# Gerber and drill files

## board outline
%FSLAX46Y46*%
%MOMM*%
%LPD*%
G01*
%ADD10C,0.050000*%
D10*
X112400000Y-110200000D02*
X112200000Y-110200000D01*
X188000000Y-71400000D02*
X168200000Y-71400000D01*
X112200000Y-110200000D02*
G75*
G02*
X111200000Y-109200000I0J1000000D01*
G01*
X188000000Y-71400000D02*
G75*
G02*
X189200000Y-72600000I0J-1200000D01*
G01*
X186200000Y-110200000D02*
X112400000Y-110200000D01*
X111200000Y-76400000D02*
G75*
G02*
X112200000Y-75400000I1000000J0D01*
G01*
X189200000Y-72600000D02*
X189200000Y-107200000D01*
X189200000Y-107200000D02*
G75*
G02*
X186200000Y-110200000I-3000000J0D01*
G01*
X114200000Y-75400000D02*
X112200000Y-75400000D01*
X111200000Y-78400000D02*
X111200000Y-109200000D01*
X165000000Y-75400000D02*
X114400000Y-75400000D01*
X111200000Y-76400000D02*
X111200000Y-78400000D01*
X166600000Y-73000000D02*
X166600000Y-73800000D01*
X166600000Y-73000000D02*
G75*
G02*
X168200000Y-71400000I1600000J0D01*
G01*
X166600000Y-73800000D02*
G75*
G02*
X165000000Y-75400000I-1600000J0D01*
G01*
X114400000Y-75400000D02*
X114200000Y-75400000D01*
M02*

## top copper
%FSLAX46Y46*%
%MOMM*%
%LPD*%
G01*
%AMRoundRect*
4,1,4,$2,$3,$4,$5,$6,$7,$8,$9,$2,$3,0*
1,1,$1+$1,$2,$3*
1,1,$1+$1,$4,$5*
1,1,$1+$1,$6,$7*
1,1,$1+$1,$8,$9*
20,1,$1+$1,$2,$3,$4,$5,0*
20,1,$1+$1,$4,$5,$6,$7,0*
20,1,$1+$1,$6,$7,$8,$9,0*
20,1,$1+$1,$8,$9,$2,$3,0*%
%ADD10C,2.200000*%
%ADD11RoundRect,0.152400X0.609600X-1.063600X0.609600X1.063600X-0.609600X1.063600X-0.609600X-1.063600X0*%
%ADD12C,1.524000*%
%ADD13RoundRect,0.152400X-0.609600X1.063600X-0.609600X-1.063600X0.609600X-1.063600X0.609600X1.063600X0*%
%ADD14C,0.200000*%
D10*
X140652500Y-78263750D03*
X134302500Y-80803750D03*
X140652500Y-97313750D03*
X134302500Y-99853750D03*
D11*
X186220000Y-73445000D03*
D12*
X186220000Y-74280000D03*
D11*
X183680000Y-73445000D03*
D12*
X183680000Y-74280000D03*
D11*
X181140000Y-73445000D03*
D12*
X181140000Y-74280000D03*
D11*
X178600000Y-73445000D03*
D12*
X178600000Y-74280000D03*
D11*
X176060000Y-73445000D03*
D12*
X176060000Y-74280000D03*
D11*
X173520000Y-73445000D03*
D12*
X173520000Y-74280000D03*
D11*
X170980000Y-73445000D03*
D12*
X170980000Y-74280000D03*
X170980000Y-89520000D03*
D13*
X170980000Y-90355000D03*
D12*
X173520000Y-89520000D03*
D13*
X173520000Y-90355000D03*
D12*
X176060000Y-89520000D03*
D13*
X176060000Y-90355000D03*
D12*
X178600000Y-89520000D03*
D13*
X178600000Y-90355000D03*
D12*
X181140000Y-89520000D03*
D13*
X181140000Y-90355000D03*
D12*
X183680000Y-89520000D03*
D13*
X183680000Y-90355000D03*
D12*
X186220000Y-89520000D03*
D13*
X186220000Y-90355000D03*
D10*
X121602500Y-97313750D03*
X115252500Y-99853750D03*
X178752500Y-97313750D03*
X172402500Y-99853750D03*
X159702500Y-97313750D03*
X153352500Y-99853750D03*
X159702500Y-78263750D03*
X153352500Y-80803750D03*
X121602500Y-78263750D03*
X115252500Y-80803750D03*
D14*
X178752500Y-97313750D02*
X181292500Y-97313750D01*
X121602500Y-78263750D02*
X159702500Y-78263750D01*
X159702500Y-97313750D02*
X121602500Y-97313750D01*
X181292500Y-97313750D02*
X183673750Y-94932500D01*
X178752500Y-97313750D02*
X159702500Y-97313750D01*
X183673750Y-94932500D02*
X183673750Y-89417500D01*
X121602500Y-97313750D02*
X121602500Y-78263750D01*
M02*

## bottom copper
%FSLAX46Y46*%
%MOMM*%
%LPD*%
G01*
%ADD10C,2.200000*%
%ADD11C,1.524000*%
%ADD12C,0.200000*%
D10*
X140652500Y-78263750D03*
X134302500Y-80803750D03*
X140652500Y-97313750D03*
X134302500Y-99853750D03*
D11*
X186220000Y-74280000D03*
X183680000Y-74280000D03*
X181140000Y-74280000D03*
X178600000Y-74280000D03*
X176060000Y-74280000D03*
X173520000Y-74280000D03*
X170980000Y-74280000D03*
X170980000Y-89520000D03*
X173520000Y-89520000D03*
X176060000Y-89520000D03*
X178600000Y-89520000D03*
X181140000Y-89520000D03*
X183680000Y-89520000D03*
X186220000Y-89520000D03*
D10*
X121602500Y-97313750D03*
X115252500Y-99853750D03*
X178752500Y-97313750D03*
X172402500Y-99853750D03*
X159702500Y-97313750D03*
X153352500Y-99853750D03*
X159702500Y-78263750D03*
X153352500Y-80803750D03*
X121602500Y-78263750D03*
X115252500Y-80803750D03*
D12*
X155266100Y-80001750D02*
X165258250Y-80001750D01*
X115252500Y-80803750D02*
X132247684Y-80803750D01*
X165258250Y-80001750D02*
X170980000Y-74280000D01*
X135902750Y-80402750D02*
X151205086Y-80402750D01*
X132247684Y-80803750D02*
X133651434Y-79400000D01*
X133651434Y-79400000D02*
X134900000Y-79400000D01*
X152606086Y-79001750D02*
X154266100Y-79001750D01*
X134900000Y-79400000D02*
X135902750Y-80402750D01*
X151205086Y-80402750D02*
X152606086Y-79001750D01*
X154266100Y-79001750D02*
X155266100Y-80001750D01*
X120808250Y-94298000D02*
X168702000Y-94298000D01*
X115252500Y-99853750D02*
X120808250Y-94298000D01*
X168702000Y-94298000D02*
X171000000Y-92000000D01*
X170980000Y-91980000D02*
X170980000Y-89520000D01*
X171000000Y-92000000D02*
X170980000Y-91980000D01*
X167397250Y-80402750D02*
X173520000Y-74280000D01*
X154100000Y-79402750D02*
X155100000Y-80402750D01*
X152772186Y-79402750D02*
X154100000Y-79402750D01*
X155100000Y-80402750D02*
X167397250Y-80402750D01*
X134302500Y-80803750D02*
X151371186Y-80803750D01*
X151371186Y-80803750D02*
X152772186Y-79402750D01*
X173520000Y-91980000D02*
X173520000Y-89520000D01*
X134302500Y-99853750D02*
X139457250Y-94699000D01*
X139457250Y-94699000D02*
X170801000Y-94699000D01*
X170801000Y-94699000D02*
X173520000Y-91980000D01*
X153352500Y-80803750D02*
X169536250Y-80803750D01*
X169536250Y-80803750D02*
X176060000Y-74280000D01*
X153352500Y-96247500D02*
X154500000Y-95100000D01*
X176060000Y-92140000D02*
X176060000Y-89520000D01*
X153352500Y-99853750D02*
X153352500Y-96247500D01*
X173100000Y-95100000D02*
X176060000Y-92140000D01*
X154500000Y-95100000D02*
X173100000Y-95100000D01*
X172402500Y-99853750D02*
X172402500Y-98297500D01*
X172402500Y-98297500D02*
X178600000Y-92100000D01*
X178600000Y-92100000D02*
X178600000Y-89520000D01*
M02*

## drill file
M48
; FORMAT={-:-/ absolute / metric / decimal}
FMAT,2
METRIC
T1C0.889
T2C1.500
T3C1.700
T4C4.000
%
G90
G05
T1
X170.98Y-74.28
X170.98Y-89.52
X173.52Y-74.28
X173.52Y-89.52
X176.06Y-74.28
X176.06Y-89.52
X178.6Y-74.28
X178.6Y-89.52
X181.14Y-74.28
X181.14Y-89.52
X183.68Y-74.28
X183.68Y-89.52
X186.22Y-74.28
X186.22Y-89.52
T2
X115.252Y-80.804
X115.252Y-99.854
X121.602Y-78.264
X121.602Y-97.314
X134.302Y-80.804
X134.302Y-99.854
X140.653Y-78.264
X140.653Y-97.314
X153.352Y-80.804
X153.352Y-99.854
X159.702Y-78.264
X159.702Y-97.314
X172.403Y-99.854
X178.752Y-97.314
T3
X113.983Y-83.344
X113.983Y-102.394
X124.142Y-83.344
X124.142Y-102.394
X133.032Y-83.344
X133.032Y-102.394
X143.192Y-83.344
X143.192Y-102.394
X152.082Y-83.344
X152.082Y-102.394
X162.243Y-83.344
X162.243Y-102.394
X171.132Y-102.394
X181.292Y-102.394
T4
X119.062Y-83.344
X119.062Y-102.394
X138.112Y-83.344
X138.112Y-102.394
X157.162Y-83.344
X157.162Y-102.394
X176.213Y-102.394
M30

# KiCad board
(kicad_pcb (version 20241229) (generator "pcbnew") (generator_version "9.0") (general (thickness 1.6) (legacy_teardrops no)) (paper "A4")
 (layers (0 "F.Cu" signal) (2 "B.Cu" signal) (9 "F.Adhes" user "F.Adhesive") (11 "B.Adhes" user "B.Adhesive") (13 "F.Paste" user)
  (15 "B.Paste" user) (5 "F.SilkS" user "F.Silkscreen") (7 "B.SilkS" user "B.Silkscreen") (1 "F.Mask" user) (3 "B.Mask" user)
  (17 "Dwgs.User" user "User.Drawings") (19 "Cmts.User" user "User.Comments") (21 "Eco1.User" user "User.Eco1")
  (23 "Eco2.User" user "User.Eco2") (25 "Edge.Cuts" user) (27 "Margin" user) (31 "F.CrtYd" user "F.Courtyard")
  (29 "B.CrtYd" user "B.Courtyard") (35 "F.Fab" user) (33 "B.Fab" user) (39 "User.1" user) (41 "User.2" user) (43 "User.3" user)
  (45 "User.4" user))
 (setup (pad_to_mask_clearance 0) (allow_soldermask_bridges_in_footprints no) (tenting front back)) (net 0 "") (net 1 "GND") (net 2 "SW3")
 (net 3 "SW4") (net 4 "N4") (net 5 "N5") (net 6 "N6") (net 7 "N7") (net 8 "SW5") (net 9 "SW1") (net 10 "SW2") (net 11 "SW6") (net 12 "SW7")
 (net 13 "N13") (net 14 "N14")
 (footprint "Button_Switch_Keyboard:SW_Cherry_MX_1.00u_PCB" (layer "F.Cu") (at 140.6525 78.26375)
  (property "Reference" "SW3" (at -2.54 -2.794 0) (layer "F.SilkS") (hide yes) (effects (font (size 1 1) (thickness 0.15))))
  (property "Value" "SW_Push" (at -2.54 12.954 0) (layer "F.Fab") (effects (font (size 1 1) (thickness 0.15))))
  (pad "" np_thru_hole circle (at -7.62 5.08) (size 1.7 1.7) (drill 1.7) (layers "*.Cu" "*.Mask"))
  (pad "" np_thru_hole circle (at -2.54 5.08) (size 4 4) (drill 4) (layers "*.Cu" "*.Mask"))
  (pad "" np_thru_hole circle (at 2.54 5.08) (size 1.7 1.7) (drill 1.7) (layers "*.Cu" "*.Mask"))
  (pad "1" thru_hole circle (at 0 0) (size 2.2 2.2) (drill 1.5) (layers "*.Cu" "*.Mask") (remove_unused_layers no) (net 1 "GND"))
  (pad "2" thru_hole circle (at -6.35 2.54) (size 2.2 2.2) (drill 1.5) (layers "*.Cu" "*.Mask") (remove_unused_layers no) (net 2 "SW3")))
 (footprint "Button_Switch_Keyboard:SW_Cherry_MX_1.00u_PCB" (layer "F.Cu") (at 140.6525 97.31375)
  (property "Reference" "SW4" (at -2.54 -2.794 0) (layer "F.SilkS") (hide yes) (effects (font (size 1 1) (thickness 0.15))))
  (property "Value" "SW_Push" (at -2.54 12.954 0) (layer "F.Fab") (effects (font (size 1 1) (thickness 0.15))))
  (pad "" np_thru_hole circle (at -7.62 5.08) (size 1.7 1.7) (drill 1.7) (layers "*.Cu" "*.Mask"))
  (pad "" np_thru_hole circle (at -2.54 5.08) (size 4 4) (drill 4) (layers "*.Cu" "*.Mask"))
  (pad "" np_thru_hole circle (at 2.54 5.08) (size 1.7 1.7) (drill 1.7) (layers "*.Cu" "*.Mask"))
  (pad "1" thru_hole circle (at 0 0) (size 2.2 2.2) (drill 1.5) (layers "*.Cu" "*.Mask") (remove_unused_layers no) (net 1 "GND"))
  (pad "2" thru_hole circle (at -6.35 2.54) (size 2.2 2.2) (drill 1.5) (layers "*.Cu" "*.Mask") (remove_unused_layers no) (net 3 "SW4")))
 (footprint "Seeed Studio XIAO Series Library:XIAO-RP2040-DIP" (layer "F.Cu") (at 178.6 81.9 -90)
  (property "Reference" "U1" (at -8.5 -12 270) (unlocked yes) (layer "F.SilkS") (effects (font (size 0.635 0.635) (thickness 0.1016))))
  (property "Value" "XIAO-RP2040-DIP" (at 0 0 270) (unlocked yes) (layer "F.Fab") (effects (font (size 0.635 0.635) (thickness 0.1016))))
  (pad "1" smd roundrect (at -8.455 -7.62 90) (size 2.432 1.524) (layers "F.Cu" "F.Mask") (roundrect_rratio 0.1) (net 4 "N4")
   (thermal_bridge_angle 45))
  (pad "1" thru_hole circle (at -7.62 -7.62 90) (size 1.524 1.524) (drill 0.889) (layers "*.Cu" "*.Mask") (remove_unused_layers no)
   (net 4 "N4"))
  (pad "2" smd roundrect (at -8.455 -5.08 90) (size 2.432 1.524) (layers "F.Cu" "F.Mask") (roundrect_rratio 0.1) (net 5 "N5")
   (thermal_bridge_angle 45))
  (pad "2" thru_hole circle (at -7.62 -5.08 90) (size 1.524 1.524) (drill 0.889) (layers "*.Cu" "*.Mask") (remove_unused_layers no)
   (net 5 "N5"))
  (pad "3" smd roundrect (at -8.455 -2.54 90) (size 2.432 1.524) (layers "F.Cu" "F.Mask") (roundrect_rratio 0.1) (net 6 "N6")
   (thermal_bridge_angle 45))
  (pad "3" thru_hole circle (at -7.62 -2.54 90) (size 1.524 1.524) (drill 0.889) (layers "*.Cu" "*.Mask") (remove_unused_layers no)
   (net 6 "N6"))
  (pad "4" smd roundrect (at -8.455 0 90) (size 2.432 1.524) (layers "F.Cu" "F.Mask") (roundrect_rratio 0.1) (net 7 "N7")
   (thermal_bridge_angle 45))
  (pad "4" thru_hole circle (at -7.62 0 90) (size 1.524 1.524) (drill 0.889) (layers "*.Cu" "*.Mask") (remove_unused_layers no) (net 7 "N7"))
  (pad "5" smd roundrect (at -8.455 2.54 90) (size 2.432 1.524) (layers "F.Cu" "F.Mask") (roundrect_rratio 0.1) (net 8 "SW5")
   (thermal_bridge_angle 45))
  (pad "5" thru_hole circle (at -7.62 2.54 90) (size 1.524 1.524) (drill 0.889) (layers "*.Cu" "*.Mask") (remove_unused_layers no)
   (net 8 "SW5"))
  (pad "6" smd roundrect (at -8.455 5.08 90) (size 2.432 1.524) (layers "F.Cu" "F.Mask") (roundrect_rratio 0.1) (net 2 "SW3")
   (thermal_bridge_angle 45))
  (pad "6" thru_hole circle (at -7.62 5.08 90) (size 1.524 1.524) (drill 0.889) (layers "*.Cu" "*.Mask") (remove_unused_layers no)
   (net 2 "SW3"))
  (pad "7" smd roundrect (at -8.455 7.62 90) (size 2.432 1.524) (layers "F.Cu" "F.Mask") (roundrect_rratio 0.1) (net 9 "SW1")
   (thermal_bridge_angle 45))
  (pad "7" thru_hole circle (at -7.62 7.62 90) (size 1.524 1.524) (drill 0.889) (layers "*.Cu" "*.Mask") (remove_unused_layers no)
   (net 9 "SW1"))
  (pad "8" thru_hole circle (at 7.62 7.62 270) (size 1.524 1.524) (drill 0.889) (layers "*.Cu" "*.Mask") (remove_unused_layers no)
   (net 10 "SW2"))
  (pad "8" smd roundrect (at 8.455 7.62 270) (size 2.432 1.524) (layers "F.Cu" "F.Mask") (roundrect_rratio 0.1) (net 10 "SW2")
   (thermal_bridge_angle 45))
  (pad "9" thru_hole circle (at 7.62 5.08 270) (size 1.524 1.524) (drill 0.889) (layers "*.Cu" "*.Mask") (remove_unused_layers no)
   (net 3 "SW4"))
  (pad "9" smd roundrect (at 8.455 5.08 270) (size 2.432 1.524) (layers "F.Cu" "F.Mask") (roundrect_rratio 0.1) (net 3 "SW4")
   (thermal_bridge_angle 45))
  (pad "10" thru_hole circle (at 7.62 2.54 270) (size 1.524 1.524) (drill 0.889) (layers "*.Cu" "*.Mask") (remove_unused_layers no)
   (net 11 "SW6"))
  (pad "10" smd roundrect (at 8.455 2.54 270) (size 2.432 1.524) (layers "F.Cu" "F.Mask") (roundrect_rratio 0.1) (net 11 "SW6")
   (thermal_bridge_angle 45))
  (pad "11" thru_hole circle (at 7.62 0 270) (size 1.524 1.524) (drill 0.889) (layers "*.Cu" "*.Mask") (remove_unused_layers no)
   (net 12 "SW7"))
  (pad "11" smd roundrect (at 8.455 0 270) (size 2.432 1.524) (layers "F.Cu" "F.Mask") (roundrect_rratio 0.1) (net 12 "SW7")
   (thermal_bridge_angle 45))
  (pad "12" thru_hole circle (at 7.62 -2.54 270) (size 1.524 1.524) (drill 0.889) (layers "*.Cu" "*.Mask") (remove_unused_layers no)
   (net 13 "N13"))
  (pad "12" smd roundrect (at 8.455 -2.54 270) (size 2.432 1.524) (layers "F.Cu" "F.Mask") (roundrect_rratio 0.1) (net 13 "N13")
   (thermal_bridge_angle 45))
  (pad "13" thru_hole circle (at 7.62 -5.08 270) (size 1.524 1.524) (drill 0.889) (layers "*.Cu" "*.Mask") (remove_unused_layers no)
   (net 1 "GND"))
  (pad "13" smd roundrect (at 8.455 -5.08 270) (size 2.432 1.524) (layers "F.Cu" "F.Mask") (roundrect_rratio 0.1) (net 1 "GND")
   (thermal_bridge_angle 45))
  (pad "14" thru_hole circle (at 7.62 -7.62 270) (size 1.524 1.524) (drill 0.889) (layers "*.Cu" "*.Mask") (remove_unused_layers no)
   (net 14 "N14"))
  (pad "14" smd roundrect (at 8.455 -7.62 270) (size 2.432 1.524) (layers "F.Cu" "F.Mask") (roundrect_rratio 0.1) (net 14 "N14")
   (thermal_bridge_angle 45)))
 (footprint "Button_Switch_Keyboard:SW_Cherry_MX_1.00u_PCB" (layer "F.Cu") (at 121.6025 97.31375)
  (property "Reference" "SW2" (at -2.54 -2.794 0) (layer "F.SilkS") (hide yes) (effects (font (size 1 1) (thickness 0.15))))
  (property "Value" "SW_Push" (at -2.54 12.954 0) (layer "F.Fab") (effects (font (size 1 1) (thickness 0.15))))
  (pad "" np_thru_hole circle (at -7.62 5.08) (size 1.7 1.7) (drill 1.7) (layers "*.Cu" "*.Mask"))
  (pad "" np_thru_hole circle (at -2.54 5.08) (size 4 4) (drill 4) (layers "*.Cu" "*.Mask"))
  (pad "" np_thru_hole circle (at 2.54 5.08) (size 1.7 1.7) (drill 1.7) (layers "*.Cu" "*.Mask"))
  (pad "1" thru_hole circle (at 0 0) (size 2.2 2.2) (drill 1.5) (layers "*.Cu" "*.Mask") (remove_unused_layers no) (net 1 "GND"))
  (pad "2" thru_hole circle (at -6.35 2.54) (size 2.2 2.2) (drill 1.5) (layers "*.Cu" "*.Mask") (remove_unused_layers no) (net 10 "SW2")))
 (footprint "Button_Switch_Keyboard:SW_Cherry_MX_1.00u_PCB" (layer "F.Cu") (at 178.7525 97.31375)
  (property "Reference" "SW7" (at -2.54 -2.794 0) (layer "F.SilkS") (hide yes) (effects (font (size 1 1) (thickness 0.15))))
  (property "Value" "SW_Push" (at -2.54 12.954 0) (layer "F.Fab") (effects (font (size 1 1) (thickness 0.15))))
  (pad "" np_thru_hole circle (at -7.62 5.08) (size 1.7 1.7) (drill 1.7) (layers "*.Cu" "*.Mask"))
  (pad "" np_thru_hole circle (at -2.54 5.08) (size 4 4) (drill 4) (layers "*.Cu" "*.Mask"))
  (pad "" np_thru_hole circle (at 2.54 5.08) (size 1.7 1.7) (drill 1.7) (layers "*.Cu" "*.Mask"))
  (pad "1" thru_hole circle (at 0 0) (size 2.2 2.2) (drill 1.5) (layers "*.Cu" "*.Mask") (remove_unused_layers no) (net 1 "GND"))
  (pad "2" thru_hole circle (at -6.35 2.54) (size 2.2 2.2) (drill 1.5) (layers "*.Cu" "*.Mask") (remove_unused_layers no) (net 12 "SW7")))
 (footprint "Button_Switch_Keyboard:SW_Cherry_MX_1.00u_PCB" (layer "F.Cu") (at 159.7025 97.31375)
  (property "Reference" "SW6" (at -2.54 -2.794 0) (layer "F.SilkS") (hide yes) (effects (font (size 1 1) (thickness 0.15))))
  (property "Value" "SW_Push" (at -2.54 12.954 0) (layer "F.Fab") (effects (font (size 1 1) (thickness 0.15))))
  (pad "" np_thru_hole circle (at -7.62 5.08) (size 1.7 1.7) (drill 1.7) (layers "*.Cu" "*.Mask"))
  (pad "" np_thru_hole circle (at -2.54 5.08) (size 4 4) (drill 4) (layers "*.Cu" "*.Mask"))
  (pad "" np_thru_hole circle (at 2.54 5.08) (size 1.7 1.7) (drill 1.7) (layers "*.Cu" "*.Mask"))
  (pad "1" thru_hole circle (at 0 0) (size 2.2 2.2) (drill 1.5) (layers "*.Cu" "*.Mask") (remove_unused_layers no) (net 1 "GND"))
  (pad "2" thru_hole circle (at -6.35 2.54) (size 2.2 2.2) (drill 1.5) (layers "*.Cu" "*.Mask") (remove_unused_layers no) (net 11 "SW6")))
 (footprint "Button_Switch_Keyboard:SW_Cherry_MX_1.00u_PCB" (layer "F.Cu") (at 159.7025 78.26375)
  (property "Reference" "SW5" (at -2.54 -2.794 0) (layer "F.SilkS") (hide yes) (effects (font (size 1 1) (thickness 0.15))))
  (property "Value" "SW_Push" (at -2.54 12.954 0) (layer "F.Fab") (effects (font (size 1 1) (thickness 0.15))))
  (pad "" np_thru_hole circle (at -7.62 5.08) (size 1.7 1.7) (drill 1.7) (layers "*.Cu" "*.Mask"))
  (pad "" np_thru_hole circle (at -2.54 5.08) (size 4 4) (drill 4) (layers "*.Cu" "*.Mask"))
  (pad "" np_thru_hole circle (at 2.54 5.08) (size 1.7 1.7) (drill 1.7) (layers "*.Cu" "*.Mask"))
  (pad "1" thru_hole circle (at 0 0) (size 2.2 2.2) (drill 1.5) (layers "*.Cu" "*.Mask") (remove_unused_layers no) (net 1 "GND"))
  (pad "2" thru_hole circle (at -6.35 2.54) (size 2.2 2.2) (drill 1.5) (layers "*.Cu" "*.Mask") (remove_unused_layers no) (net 8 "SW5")))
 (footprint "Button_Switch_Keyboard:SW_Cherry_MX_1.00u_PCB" (layer "F.Cu") (at 121.6025 78.26375)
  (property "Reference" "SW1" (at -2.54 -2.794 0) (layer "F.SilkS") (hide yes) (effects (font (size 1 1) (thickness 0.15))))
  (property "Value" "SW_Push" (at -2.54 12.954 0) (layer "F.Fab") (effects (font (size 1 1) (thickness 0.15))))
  (pad "" np_thru_hole circle (at -7.62 5.08) (size 1.7 1.7) (drill 1.7) (layers "*.Cu" "*.Mask"))
  (pad "" np_thru_hole circle (at -2.54 5.08) (size 4 4) (drill 4) (layers "*.Cu" "*.Mask"))
  (pad "" np_thru_hole circle (at 2.54 5.08) (size 1.7 1.7) (drill 1.7) (layers "*.Cu" "*.Mask"))
  (pad "1" thru_hole circle (at 0 0) (size 2.2 2.2) (drill 1.5) (layers "*.Cu" "*.Mask") (remove_unused_layers no) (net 1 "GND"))
  (pad "2" thru_hole circle (at -6.35 2.54) (size 2.2 2.2) (drill 1.5) (layers "*.Cu" "*.Mask") (remove_unused_layers no) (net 9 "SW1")))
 (gr_line (start 112.4 110.2) (end 112.2 110.2) (stroke (width 0.05) (type default)) (layer "Edge.Cuts"))
 (gr_line (start 188 71.4) (end 168.2 71.4) (stroke (width 0.05) (type default)) (layer "Edge.Cuts"))
 (gr_arc (start 112.2 110.2) (mid 111.492893 109.907107) (end 111.2 109.2) (stroke (width 0.05) (type default)) (layer "Edge.Cuts"))
 (gr_arc (start 188 71.4) (mid 188.848528 71.751472) (end 189.2 72.6) (stroke (width 0.05) (type default)) (layer "Edge.Cuts"))
 (gr_line (start 186.2 110.2) (end 112.4 110.2) (stroke (width 0.05) (type default)) (layer "Edge.Cuts"))
 (gr_arc (start 111.2 76.4) (mid 111.492893 75.692893) (end 112.2 75.4) (stroke (width 0.05) (type default)) (layer "Edge.Cuts"))
 (gr_line (start 189.2 72.6) (end 189.2 107.2) (stroke (width 0.05) (type default)) (layer "Edge.Cuts"))
 (gr_arc (start 189.2 107.2) (mid 188.32132 109.32132) (end 186.2 110.2) (stroke (width 0.05) (type default)) (layer "Edge.Cuts"))
 (gr_line (start 114.2 75.4) (end 112.2 75.4) (stroke (width 0.05) (type default)) (layer "Edge.Cuts"))
 (gr_line (start 111.2 78.4) (end 111.2 109.2) (stroke (width 0.05) (type default)) (layer "Edge.Cuts"))
 (gr_line (start 165 75.4) (end 114.4 75.4) (stroke (width 0.05) (type default)) (layer "Edge.Cuts"))
 (gr_line (start 111.2 76.4) (end 111.2 78.4) (stroke (width 0.05) (type default)) (layer "Edge.Cuts"))
 (gr_line (start 166.6 73) (end 166.6 73.8) (stroke (width 0.05) (type default)) (layer "Edge.Cuts"))
 (gr_arc (start 166.6 73) (mid 167.068629 71.868629) (end 168.2 71.4) (stroke (width 0.05) (type default)) (layer "Edge.Cuts"))
 (gr_arc (start 166.6 73.8) (mid 166.131371 74.931371) (end 165 75.4) (stroke (width 0.05) (type default)) (layer "Edge.Cuts"))
 (gr_line (start 114.4 75.4) (end 114.2 75.4) (stroke (width 0.05) (type default)) (layer "Edge.Cuts"))
 (segment (start 178.7525 97.31375) (end 181.2925 97.31375) (width 0.2) (layer "F.Cu") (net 1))
 (segment (start 121.6025 78.26375) (end 159.7025 78.26375) (width 0.2) (layer "F.Cu") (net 1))
 (segment (start 159.7025 97.31375) (end 121.6025 97.31375) (width 0.2) (layer "F.Cu") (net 1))
 (segment (start 181.2925 97.31375) (end 183.67375 94.9325) (width 0.2) (layer "F.Cu") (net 1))
 (segment (start 178.7525 97.31375) (end 159.7025 97.31375) (width 0.2) (layer "F.Cu") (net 1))
 (segment (start 183.67375 94.9325) (end 183.67375 89.4175) (width 0.2) (layer "F.Cu") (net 1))
 (segment (start 121.6025 97.31375) (end 121.6025 78.26375) (width 0.2) (layer "F.Cu") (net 1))
 (segment (start 155.2661 80.00175) (end 165.25825 80.00175) (width 0.2) (layer "B.Cu") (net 9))
 (segment (start 115.2525 80.80375) (end 132.247684 80.80375) (width 0.2) (layer "B.Cu") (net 9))
 (segment (start 165.25825 80.00175) (end 170.98 74.28) (width 0.2) (layer "B.Cu") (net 9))
 (segment (start 135.90275 80.40275) (end 151.205086 80.40275) (width 0.2) (layer "B.Cu") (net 9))
 (segment (start 132.247684 80.80375) (end 133.651434 79.4) (width 0.2) (layer "B.Cu") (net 9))
 (segment (start 133.651434 79.4) (end 134.9 79.4) (width 0.2) (layer "B.Cu") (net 9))
 (segment (start 152.606086 79.00175) (end 154.2661 79.00175) (width 0.2) (layer "B.Cu") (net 9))
 (segment (start 134.9 79.4) (end 135.90275 80.40275) (width 0.2) (layer "B.Cu") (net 9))
 (segment (start 151.205086 80.40275) (end 152.606086 79.00175) (width 0.2) (layer "B.Cu") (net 9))
 (segment (start 154.2661 79.00175) (end 155.2661 80.00175) (width 0.2) (layer "B.Cu") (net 9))
 (segment (start 120.80825 94.298) (end 168.702 94.298) (width 0.2) (layer "B.Cu") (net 10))
 (segment (start 115.2525 99.85375) (end 120.80825 94.298) (width 0.2) (layer "B.Cu") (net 10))
 (segment (start 168.702 94.298) (end 171 92) (width 0.2) (layer "B.Cu") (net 10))
 (segment (start 170.98 91.98) (end 170.98 89.52) (width 0.2) (layer "B.Cu") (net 10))
 (segment (start 171 92) (end 170.98 91.98) (width 0.2) (layer "B.Cu") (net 10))
 (segment (start 167.39725 80.40275) (end 173.52 74.28) (width 0.2) (layer "B.Cu") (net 2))
 (segment (start 154.1 79.40275) (end 155.1 80.40275) (width 0.2) (layer "B.Cu") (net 2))
 (segment (start 152.772186 79.40275) (end 154.1 79.40275) (width 0.2) (layer "B.Cu") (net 2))
 (segment (start 155.1 80.40275) (end 167.39725 80.40275) (width 0.2) (layer "B.Cu") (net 2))
 (segment (start 134.3025 80.80375) (end 151.371186 80.80375) (width 0.2) (layer "B.Cu") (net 2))
 (segment (start 151.371186 80.80375) (end 152.772186 79.40275) (width 0.2) (layer "B.Cu") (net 2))
 (segment (start 173.52 91.98) (end 173.52 89.52) (width 0.2) (layer "B.Cu") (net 3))
 (segment (start 134.3025 99.85375) (end 139.45725 94.699) (width 0.2) (layer "B.Cu") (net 3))
 (segment (start 139.45725 94.699) (end 170.801 94.699) (width 0.2) (layer "B.Cu") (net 3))
 (segment (start 170.801 94.699) (end 173.52 91.98) (width 0.2) (layer "B.Cu") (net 3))
 (segment (start 153.3525 80.80375) (end 169.53625 80.80375) (width 0.2) (layer "B.Cu") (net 8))
 (segment (start 169.53625 80.80375) (end 176.06 74.28) (width 0.2) (layer "B.Cu") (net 8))
 (segment (start 153.3525 96.2475) (end 154.5 95.1) (width 0.2) (layer "B.Cu") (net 11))
 (segment (start 176.06 92.14) (end 176.06 89.52) (width 0.2) (layer "B.Cu") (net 11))
 (segment (start 153.3525 99.85375) (end 153.3525 96.2475) (width 0.2) (layer "B.Cu") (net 11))
 (segment (start 173.1 95.1) (end 176.06 92.14) (width 0.2) (layer "B.Cu") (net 11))
 (segment (start 154.5 95.1) (end 173.1 95.1) (width 0.2) (layer "B.Cu") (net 11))
 (segment (start 172.4025 99.85375) (end 172.4025 98.2975) (width 0.2) (layer "B.Cu") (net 12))
 (segment (start 172.4025 98.2975) (end 178.6 92.1) (width 0.2) (layer "B.Cu") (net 12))
 (segment (start 178.6 92.1) (end 178.6 89.52) (width 0.2) (layer "B.Cu") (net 12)))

